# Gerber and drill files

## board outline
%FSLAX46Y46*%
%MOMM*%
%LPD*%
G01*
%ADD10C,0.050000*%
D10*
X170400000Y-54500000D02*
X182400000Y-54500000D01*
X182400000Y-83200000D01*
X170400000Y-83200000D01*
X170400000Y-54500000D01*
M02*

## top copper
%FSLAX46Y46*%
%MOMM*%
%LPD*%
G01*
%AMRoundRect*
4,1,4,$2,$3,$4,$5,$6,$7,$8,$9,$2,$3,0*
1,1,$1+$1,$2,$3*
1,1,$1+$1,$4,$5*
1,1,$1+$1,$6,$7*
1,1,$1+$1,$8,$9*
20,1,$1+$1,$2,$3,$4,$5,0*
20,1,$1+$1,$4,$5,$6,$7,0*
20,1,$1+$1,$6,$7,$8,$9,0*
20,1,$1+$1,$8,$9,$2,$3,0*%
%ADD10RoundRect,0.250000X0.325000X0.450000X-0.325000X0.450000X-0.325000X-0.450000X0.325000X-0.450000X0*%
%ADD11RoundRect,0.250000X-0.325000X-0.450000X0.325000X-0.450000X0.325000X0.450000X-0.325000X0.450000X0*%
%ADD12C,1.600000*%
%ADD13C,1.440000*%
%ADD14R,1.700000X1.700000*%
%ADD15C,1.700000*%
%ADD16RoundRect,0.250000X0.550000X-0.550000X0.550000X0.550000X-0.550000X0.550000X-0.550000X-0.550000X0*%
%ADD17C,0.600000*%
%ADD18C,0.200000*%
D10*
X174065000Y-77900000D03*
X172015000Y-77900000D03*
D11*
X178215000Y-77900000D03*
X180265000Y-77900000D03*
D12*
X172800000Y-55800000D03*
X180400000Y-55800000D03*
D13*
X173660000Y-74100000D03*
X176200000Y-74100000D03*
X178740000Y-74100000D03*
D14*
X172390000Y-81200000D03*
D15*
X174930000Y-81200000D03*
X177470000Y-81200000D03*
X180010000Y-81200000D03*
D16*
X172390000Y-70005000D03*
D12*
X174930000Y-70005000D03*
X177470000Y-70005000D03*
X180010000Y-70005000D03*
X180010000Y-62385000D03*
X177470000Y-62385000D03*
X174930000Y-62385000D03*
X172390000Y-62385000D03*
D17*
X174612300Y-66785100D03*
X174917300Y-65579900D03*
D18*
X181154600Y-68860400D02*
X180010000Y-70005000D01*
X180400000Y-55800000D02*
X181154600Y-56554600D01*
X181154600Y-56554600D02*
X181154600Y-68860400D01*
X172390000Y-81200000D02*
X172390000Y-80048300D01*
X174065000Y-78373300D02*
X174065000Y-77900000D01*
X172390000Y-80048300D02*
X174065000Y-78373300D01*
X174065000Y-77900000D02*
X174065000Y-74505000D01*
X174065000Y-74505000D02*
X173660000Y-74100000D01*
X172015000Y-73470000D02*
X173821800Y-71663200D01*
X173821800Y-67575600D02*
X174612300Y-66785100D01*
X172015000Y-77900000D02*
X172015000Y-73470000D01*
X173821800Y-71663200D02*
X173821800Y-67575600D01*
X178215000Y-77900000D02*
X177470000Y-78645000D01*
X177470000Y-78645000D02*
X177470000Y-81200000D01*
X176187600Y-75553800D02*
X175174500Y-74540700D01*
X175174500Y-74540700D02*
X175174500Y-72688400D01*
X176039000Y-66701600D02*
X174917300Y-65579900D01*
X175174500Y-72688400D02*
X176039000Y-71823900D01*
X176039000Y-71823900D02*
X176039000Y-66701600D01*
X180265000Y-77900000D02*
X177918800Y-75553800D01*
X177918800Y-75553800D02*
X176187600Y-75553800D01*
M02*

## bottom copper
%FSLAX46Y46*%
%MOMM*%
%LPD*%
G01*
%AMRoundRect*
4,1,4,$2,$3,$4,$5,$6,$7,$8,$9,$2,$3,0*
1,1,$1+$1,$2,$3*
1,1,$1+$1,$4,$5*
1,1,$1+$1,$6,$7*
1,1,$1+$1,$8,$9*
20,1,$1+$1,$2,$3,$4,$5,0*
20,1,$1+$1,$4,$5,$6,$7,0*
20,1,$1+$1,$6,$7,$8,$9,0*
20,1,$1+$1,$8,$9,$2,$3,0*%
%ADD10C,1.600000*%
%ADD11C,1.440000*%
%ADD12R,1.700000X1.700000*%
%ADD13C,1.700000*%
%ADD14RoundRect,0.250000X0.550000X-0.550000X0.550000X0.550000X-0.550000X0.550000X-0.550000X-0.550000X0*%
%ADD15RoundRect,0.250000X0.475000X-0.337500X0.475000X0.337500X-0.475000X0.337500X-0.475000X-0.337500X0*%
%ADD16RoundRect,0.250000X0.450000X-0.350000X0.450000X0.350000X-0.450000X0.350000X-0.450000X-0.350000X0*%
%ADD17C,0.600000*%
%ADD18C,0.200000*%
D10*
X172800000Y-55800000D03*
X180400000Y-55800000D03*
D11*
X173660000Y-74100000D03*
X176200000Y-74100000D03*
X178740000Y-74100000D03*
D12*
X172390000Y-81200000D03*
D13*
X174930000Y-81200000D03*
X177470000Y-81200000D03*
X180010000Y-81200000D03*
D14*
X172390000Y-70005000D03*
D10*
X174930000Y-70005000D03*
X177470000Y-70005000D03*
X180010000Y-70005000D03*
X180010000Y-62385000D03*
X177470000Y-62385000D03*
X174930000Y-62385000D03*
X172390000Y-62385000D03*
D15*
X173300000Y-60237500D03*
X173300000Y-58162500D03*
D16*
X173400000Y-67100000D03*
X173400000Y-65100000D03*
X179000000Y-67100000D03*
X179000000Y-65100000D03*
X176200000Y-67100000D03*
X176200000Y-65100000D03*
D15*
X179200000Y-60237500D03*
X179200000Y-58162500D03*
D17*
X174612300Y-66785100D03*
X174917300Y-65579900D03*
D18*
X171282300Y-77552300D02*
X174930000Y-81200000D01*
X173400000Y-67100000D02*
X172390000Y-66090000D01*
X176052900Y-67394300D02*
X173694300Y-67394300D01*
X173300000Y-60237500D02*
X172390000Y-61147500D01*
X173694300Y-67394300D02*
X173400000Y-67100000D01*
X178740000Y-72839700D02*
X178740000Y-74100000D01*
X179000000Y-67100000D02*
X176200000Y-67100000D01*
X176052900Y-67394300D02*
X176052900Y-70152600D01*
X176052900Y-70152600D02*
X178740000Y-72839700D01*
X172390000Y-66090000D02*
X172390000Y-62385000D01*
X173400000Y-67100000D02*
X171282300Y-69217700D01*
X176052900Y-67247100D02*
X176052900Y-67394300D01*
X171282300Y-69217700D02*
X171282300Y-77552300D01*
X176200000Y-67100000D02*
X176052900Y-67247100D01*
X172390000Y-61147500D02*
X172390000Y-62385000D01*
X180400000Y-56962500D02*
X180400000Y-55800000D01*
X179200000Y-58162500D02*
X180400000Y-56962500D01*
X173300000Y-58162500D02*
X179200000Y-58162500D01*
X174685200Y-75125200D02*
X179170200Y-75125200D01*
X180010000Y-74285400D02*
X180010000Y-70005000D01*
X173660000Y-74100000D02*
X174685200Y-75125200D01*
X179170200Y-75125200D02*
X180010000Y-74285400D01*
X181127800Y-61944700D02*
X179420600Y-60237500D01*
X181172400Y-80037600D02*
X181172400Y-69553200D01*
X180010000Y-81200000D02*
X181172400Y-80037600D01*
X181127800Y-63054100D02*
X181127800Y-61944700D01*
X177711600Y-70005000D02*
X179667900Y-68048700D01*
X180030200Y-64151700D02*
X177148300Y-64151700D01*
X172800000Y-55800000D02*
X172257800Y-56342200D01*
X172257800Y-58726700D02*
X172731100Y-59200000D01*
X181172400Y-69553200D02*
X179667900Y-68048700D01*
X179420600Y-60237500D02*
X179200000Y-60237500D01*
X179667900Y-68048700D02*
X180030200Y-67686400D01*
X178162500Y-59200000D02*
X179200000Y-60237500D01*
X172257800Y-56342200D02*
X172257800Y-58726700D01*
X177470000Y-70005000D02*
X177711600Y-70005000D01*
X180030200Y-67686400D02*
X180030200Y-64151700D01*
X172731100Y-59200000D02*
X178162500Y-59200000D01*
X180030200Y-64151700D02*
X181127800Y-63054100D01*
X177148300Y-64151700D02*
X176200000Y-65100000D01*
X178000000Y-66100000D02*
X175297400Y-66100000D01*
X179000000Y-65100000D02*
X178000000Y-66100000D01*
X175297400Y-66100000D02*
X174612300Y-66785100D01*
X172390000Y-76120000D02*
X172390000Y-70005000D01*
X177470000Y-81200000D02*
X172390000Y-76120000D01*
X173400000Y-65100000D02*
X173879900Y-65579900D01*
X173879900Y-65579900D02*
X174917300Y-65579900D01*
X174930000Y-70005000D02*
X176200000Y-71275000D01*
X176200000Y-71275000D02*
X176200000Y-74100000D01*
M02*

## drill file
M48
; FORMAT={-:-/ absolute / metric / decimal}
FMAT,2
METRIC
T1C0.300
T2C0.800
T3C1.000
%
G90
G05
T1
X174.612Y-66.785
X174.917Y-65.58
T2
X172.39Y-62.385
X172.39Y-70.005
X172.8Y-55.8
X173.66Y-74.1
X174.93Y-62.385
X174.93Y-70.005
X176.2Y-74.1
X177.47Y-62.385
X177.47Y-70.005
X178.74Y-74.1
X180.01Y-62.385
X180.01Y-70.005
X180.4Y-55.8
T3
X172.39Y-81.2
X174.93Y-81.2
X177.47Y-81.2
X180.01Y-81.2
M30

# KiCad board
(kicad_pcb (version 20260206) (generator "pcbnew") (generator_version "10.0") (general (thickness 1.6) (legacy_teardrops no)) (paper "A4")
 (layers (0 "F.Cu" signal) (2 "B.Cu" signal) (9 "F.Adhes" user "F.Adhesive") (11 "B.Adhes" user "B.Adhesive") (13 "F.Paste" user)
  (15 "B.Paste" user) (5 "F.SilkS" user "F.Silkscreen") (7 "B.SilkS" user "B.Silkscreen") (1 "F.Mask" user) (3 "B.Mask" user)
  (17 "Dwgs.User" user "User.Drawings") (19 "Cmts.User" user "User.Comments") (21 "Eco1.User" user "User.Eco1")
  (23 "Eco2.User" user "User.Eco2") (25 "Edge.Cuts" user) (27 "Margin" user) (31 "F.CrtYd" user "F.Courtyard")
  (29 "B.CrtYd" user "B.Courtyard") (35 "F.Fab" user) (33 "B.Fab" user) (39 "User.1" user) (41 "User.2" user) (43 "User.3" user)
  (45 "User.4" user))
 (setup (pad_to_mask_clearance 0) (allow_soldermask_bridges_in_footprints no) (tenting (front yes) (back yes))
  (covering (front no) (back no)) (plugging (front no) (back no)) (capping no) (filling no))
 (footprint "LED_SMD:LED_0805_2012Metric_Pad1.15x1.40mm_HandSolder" (layer "F.Cu") (at 173.04 77.9 180)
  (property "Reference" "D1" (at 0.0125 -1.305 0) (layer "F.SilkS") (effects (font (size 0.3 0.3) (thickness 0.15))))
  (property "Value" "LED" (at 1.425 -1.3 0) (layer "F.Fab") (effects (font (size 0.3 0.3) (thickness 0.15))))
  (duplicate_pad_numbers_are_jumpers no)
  (pad "1" smd roundrect (at -1.025 0 180) (size 1.15 1.4) (layers "F.Cu" "F.Mask" "F.Paste") (roundrect_rratio 0.217391) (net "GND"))
  (pad "2" smd roundrect (at 1.025 0 180) (size 1.15 1.4) (layers "F.Cu" "F.Mask" "F.Paste") (roundrect_rratio 0.217391) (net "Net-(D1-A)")))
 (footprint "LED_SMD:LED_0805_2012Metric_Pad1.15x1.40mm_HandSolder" (layer "F.Cu") (at 179.24 77.9)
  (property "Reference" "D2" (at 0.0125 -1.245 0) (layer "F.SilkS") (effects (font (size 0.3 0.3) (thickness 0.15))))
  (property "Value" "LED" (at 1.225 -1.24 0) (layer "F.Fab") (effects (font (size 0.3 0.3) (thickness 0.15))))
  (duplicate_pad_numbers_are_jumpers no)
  (pad "1" smd roundrect (at -1.025 0) (size 1.15 1.4) (layers "F.Cu" "F.Mask" "F.Paste") (roundrect_rratio 0.217391) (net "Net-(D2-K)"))
  (pad "2" smd roundrect (at 1.025 0) (size 1.15 1.4) (layers "F.Cu" "F.Mask" "F.Paste") (roundrect_rratio 0.217391) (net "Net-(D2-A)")))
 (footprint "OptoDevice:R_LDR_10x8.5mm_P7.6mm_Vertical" (layer "F.Cu") (at 172.8 55.8)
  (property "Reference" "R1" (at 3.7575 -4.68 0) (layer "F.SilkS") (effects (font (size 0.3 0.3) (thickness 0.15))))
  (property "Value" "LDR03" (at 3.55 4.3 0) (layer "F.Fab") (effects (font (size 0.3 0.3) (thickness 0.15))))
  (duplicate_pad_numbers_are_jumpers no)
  (pad "1" thru_hole circle (at 0 0) (size 1.6 1.6) (drill 0.8) (layers "*.Cu" "*.Mask") (remove_unused_layers no) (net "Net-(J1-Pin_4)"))
  (pad "2" thru_hole circle (at 7.6 0) (size 1.6 1.6) (drill 0.8) (layers "*.Cu" "*.Mask") (remove_unused_layers no) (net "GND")))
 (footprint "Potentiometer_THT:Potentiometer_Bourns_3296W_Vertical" (layer "F.Cu") (at 173.66 74.1 180)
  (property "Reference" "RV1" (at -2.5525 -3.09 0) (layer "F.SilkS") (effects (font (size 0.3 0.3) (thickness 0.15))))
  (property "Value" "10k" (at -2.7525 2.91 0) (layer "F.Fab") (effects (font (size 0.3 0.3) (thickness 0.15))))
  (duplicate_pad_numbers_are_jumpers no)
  (pad "1" thru_hole circle (at 0 0 180) (size 1.44 1.44) (drill 0.8) (layers "*.Cu" "*.Mask") (remove_unused_layers no) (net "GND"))
  (pad "2" thru_hole circle (at -2.54 0 180) (size 1.44 1.44) (drill 0.8) (layers "*.Cu" "*.Mask") (remove_unused_layers no)
   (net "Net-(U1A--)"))
  (pad "3" thru_hole circle (at -5.08 0 180) (size 1.44 1.44) (drill 0.8) (layers "*.Cu" "*.Mask") (remove_unused_layers no) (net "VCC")))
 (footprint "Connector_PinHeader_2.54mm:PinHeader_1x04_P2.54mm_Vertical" (layer "F.Cu") (at 172.39 81.2 90)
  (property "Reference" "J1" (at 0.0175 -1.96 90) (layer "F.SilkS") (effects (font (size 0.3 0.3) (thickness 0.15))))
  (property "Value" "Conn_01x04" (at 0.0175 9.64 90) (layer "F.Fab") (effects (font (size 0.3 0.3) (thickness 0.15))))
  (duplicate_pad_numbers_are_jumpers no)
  (pad "1" thru_hole rect (at 0 0 90) (size 1.7 1.7) (drill 1) (layers "*.Cu" "*.Mask") (remove_unused_layers no) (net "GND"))
  (pad "2" thru_hole circle (at 0 2.54 90) (size 1.7 1.7) (drill 1) (layers "*.Cu" "*.Mask") (remove_unused_layers no) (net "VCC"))
  (pad "3" thru_hole circle (at 0 5.08 90) (size 1.7 1.7) (drill 1) (layers "*.Cu" "*.Mask") (remove_unused_layers no) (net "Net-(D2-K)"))
  (pad "4" thru_hole circle (at 0 7.62 90) (size 1.7 1.7) (drill 1) (layers "*.Cu" "*.Mask") (remove_unused_layers no)
   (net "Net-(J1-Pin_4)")))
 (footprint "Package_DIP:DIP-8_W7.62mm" (layer "F.Cu") (at 172.39 70.005 90)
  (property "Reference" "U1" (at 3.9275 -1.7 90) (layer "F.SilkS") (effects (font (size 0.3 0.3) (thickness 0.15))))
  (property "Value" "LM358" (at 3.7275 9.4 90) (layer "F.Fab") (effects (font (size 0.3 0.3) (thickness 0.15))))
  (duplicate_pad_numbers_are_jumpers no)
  (pad "1" thru_hole roundrect (at 0 0 90) (size 1.6 1.6) (drill 0.8) (layers "*.Cu" "*.Mask") (remove_unused_layers no)
   (roundrect_rratio 0.15625) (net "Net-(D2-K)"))
  (pad "2" thru_hole circle (at 0 2.54 90) (size 1.6 1.6) (drill 0.8) (layers "*.Cu" "*.Mask") (remove_unused_layers no) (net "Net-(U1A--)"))
  (pad "3" thru_hole circle (at 0 5.08 90) (size 1.6 1.6) (drill 0.8) (layers "*.Cu" "*.Mask") (remove_unused_layers no)
   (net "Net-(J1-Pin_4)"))
  (pad "4" thru_hole circle (at 0 7.62 90) (size 1.6 1.6) (drill 0.8) (layers "*.Cu" "*.Mask") (remove_unused_layers no) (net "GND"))
  (pad "5" thru_hole circle (at 7.62 7.62 90) (size 1.6 1.6) (drill 0.8) (layers "*.Cu" "*.Mask") (remove_unused_layers no))
  (pad "6" thru_hole circle (at 7.62 5.08 90) (size 1.6 1.6) (drill 0.8) (layers "*.Cu" "*.Mask") (remove_unused_layers no))
  (pad "7" thru_hole circle (at 7.62 2.54 90) (size 1.6 1.6) (drill 0.8) (layers "*.Cu" "*.Mask") (remove_unused_layers no))
  (pad "8" thru_hole circle (at 7.62 0 90) (size 1.6 1.6) (drill 0.8) (layers "*.Cu" "*.Mask") (remove_unused_layers no) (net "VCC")))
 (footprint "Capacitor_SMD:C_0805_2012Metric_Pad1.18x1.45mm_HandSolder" (layer "B.Cu") (at 173.3 59.2 90)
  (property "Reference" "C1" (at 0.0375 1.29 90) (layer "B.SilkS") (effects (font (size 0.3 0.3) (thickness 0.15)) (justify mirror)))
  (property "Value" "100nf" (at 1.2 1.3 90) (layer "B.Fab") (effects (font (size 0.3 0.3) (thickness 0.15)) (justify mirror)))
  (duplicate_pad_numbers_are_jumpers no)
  (pad "1" smd roundrect (at -1.0375 0 90) (size 1.175 1.45) (layers "B.Cu" "B.Mask" "B.Paste") (roundrect_rratio 0.212766) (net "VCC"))
  (pad "2" smd roundrect (at 1.0375 0 90) (size 1.175 1.45) (layers "B.Cu" "B.Mask" "B.Paste") (roundrect_rratio 0.212766) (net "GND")))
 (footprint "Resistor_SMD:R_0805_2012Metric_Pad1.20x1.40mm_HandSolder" (layer "B.Cu") (at 173.4 66.1 90)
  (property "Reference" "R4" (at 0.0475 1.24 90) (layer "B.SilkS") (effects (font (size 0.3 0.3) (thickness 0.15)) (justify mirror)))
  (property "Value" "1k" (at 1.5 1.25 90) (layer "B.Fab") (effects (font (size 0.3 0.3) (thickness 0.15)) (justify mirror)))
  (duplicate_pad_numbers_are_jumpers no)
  (pad "1" smd roundrect (at -1 0 90) (size 1.2 1.4) (layers "B.Cu" "B.Mask" "B.Paste") (roundrect_rratio 0.208333) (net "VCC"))
  (pad "2" smd roundrect (at 1 0 90) (size 1.2 1.4) (layers "B.Cu" "B.Mask" "B.Paste") (roundrect_rratio 0.208333) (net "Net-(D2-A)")))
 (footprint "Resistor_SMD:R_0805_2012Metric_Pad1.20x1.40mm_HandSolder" (layer "B.Cu") (at 179 66.1 90)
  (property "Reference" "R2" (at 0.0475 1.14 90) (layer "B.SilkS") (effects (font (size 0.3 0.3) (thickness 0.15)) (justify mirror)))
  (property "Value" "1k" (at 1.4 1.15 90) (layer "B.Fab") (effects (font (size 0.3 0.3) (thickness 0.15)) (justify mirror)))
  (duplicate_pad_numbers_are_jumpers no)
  (pad "1" smd roundrect (at -1 0 90) (size 1.2 1.4) (layers "B.Cu" "B.Mask" "B.Paste") (roundrect_rratio 0.208333) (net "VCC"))
  (pad "2" smd roundrect (at 1 0 90) (size 1.2 1.4) (layers "B.Cu" "B.Mask" "B.Paste") (roundrect_rratio 0.208333) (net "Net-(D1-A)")))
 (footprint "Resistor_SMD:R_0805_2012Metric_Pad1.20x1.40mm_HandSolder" (layer "B.Cu") (at 176.2 66.1 90)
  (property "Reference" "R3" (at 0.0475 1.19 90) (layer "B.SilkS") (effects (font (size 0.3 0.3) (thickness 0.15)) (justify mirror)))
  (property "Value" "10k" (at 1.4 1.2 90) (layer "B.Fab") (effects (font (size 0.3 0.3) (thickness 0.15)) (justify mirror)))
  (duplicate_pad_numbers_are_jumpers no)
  (pad "1" smd roundrect (at -1 0 90) (size 1.2 1.4) (layers "B.Cu" "B.Mask" "B.Paste") (roundrect_rratio 0.208333) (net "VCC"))
  (pad "2" smd roundrect (at 1 0 90) (size 1.2 1.4) (layers "B.Cu" "B.Mask" "B.Paste") (roundrect_rratio 0.208333) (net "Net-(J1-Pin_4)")))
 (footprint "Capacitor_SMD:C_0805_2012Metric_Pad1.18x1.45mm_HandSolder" (layer "B.Cu") (at 179.2 59.2 90)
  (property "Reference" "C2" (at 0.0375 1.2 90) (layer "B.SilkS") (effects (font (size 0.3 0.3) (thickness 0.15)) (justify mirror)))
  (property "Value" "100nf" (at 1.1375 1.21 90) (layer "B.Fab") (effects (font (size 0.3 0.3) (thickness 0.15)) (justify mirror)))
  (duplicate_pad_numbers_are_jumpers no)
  (pad "1" smd roundrect (at -1.0375 0 90) (size 1.175 1.45) (layers "B.Cu" "B.Mask" "B.Paste") (roundrect_rratio 0.212766)
   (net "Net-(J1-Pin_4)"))
  (pad "2" smd roundrect (at 1.0375 0 90) (size 1.175 1.45) (layers "B.Cu" "B.Mask" "B.Paste") (roundrect_rratio 0.212766) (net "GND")))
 (gr_rect (start 170.4 54.5) (end 182.4 83.2) (stroke (width 0.05) (type default)) (fill no) (layer "Edge.Cuts"))
 (segment (start 171.2823 77.5523) (end 174.93 81.2) (width 0.2) (layer "B.Cu") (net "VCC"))
 (segment (start 173.4 67.1) (end 172.39 66.09) (width 0.2) (layer "B.Cu") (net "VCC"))
 (segment (start 176.0529 67.3943) (end 173.6943 67.3943) (width 0.2) (layer "B.Cu") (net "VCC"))
 (segment (start 173.3 60.2375) (end 172.39 61.1475) (width 0.2) (layer "B.Cu") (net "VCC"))
 (segment (start 173.6943 67.3943) (end 173.4 67.1) (width 0.2) (layer "B.Cu") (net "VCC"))
 (segment (start 178.74 72.8397) (end 178.74 74.1) (width 0.2) (layer "B.Cu") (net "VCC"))
 (segment (start 179 67.1) (end 176.2 67.1) (width 0.2) (layer "B.Cu") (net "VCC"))
 (segment (start 176.0529 67.3943) (end 176.0529 70.1526) (width 0.2) (layer "B.Cu") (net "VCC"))
 (segment (start 176.0529 70.1526) (end 178.74 72.8397) (width 0.2) (layer "B.Cu") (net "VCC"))
 (segment (start 172.39 66.09) (end 172.39 62.385) (width 0.2) (layer "B.Cu") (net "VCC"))
 (segment (start 173.4 67.1) (end 171.2823 69.2177) (width 0.2) (layer "B.Cu") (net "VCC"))
 (segment (start 176.0529 67.2471) (end 176.0529 67.3943) (width 0.2) (layer "B.Cu") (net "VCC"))
 (segment (start 171.2823 69.2177) (end 171.2823 77.5523) (width 0.2) (layer "B.Cu") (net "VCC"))
 (segment (start 176.2 67.1) (end 176.0529 67.2471) (width 0.2) (layer "B.Cu") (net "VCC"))
 (segment (start 172.39 61.1475) (end 172.39 62.385) (width 0.2) (layer "B.Cu") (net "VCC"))
 (segment (start 181.1546 68.8604) (end 180.01 70.005) (width 0.2) (layer "F.Cu") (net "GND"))
 (segment (start 180.4 55.8) (end 181.1546 56.5546) (width 0.2) (layer "F.Cu") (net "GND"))
 (segment (start 181.1546 56.5546) (end 181.1546 68.8604) (width 0.2) (layer "F.Cu") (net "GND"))
 (segment (start 172.39 81.2) (end 172.39 80.0483) (width 0.2) (layer "F.Cu") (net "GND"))
 (segment (start 174.065 78.3733) (end 174.065 77.9) (width 0.2) (layer "F.Cu") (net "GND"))
 (segment (start 172.39 80.0483) (end 174.065 78.3733) (width 0.2) (layer "F.Cu") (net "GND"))
 (segment (start 174.065 77.9) (end 174.065 74.505) (width 0.2) (layer "F.Cu") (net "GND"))
 (segment (start 174.065 74.505) (end 173.66 74.1) (width 0.2) (layer "F.Cu") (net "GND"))
 (segment (start 180.4 56.9625) (end 180.4 55.8) (width 0.2) (layer "B.Cu") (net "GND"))
 (segment (start 179.2 58.1625) (end 180.4 56.9625) (width 0.2) (layer "B.Cu") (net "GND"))
 (segment (start 173.3 58.1625) (end 179.2 58.1625) (width 0.2) (layer "B.Cu") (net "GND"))
 (segment (start 174.6852 75.1252) (end 179.1702 75.1252) (width 0.2) (layer "B.Cu") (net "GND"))
 (segment (start 180.01 74.2854) (end 180.01 70.005) (width 0.2) (layer "B.Cu") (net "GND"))
 (segment (start 173.66 74.1) (end 174.6852 75.1252) (width 0.2) (layer "B.Cu") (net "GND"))
 (segment (start 179.1702 75.1252) (end 180.01 74.2854) (width 0.2) (layer "B.Cu") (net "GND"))
 (segment (start 181.1278 61.9447) (end 179.4206 60.2375) (width 0.2) (layer "B.Cu") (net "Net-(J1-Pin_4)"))
 (segment (start 181.1724 80.0376) (end 181.1724 69.5532) (width 0.2) (layer "B.Cu") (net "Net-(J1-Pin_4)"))
 (segment (start 180.01 81.2) (end 181.1724 80.0376) (width 0.2) (layer "B.Cu") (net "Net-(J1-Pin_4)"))
 (segment (start 181.1278 63.0541) (end 181.1278 61.9447) (width 0.2) (layer "B.Cu") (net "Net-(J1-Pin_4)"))
 (segment (start 177.7116 70.005) (end 179.6679 68.0487) (width 0.2) (layer "B.Cu") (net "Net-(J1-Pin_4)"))
 (segment (start 180.0302 64.1517) (end 177.1483 64.1517) (width 0.2) (layer "B.Cu") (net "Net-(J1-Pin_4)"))
 (segment (start 172.8 55.8) (end 172.2578 56.3422) (width 0.2) (layer "B.Cu") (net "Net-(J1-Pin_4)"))
 (segment (start 172.2578 58.7267) (end 172.7311 59.2) (width 0.2) (layer "B.Cu") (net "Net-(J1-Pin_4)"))
 (segment (start 181.1724 69.5532) (end 179.6679 68.0487) (width 0.2) (layer "B.Cu") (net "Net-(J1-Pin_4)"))
 (segment (start 179.4206 60.2375) (end 179.2 60.2375) (width 0.2) (layer "B.Cu") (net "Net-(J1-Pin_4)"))
 (segment (start 179.6679 68.0487) (end 180.0302 67.6864) (width 0.2) (layer "B.Cu") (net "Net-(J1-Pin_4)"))
 (segment (start 178.1625 59.2) (end 179.2 60.2375) (width 0.2) (layer "B.Cu") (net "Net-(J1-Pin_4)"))
 (segment (start 172.2578 56.3422) (end 172.2578 58.7267) (width 0.2) (layer "B.Cu") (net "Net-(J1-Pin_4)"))
 (segment (start 177.47 70.005) (end 177.7116 70.005) (width 0.2) (layer "B.Cu") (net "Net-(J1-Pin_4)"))
 (segment (start 180.0302 67.6864) (end 180.0302 64.1517) (width 0.2) (layer "B.Cu") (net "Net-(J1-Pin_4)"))
 (segment (start 172.7311 59.2) (end 178.1625 59.2) (width 0.2) (layer "B.Cu") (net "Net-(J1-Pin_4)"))
 (segment (start 180.0302 64.1517) (end 181.1278 63.0541) (width 0.2) (layer "B.Cu") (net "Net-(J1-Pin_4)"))
 (segment (start 177.1483 64.1517) (end 176.2 65.1) (width 0.2) (layer "B.Cu") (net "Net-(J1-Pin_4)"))
 (segment (start 172.015 73.47) (end 173.8218 71.6632) (width 0.2) (layer "F.Cu") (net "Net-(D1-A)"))
 (segment (start 173.8218 67.5756) (end 174.6123 66.7851) (width 0.2) (layer "F.Cu") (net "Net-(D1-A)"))
 (segment (start 172.015 77.9) (end 172.015 73.47) (width 0.2) (layer "F.Cu") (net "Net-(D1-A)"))
 (segment (start 173.8218 71.6632) (end 173.8218 67.5756) (width 0.2) (layer "F.Cu") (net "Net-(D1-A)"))
 (via (at 174.6123 66.7851) (size 0.6) (drill 0.3) (layers "F.Cu" "B.Cu") (capping no) (covering (front no) (back no))
  (plugging (front no) (back no)) (filling no) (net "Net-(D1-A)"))
 (segment (start 178 66.1) (end 175.2974 66.1) (width 0.2) (layer "B.Cu") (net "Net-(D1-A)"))
 (segment (start 179 65.1) (end 178 66.1) (width 0.2) (layer "B.Cu") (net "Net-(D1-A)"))
 (segment (start 175.2974 66.1) (end 174.6123 66.7851) (width 0.2) (layer "B.Cu") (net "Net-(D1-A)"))
 (segment (start 178.215 77.9) (end 177.47 78.645) (width 0.2) (layer "F.Cu") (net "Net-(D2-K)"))
 (segment (start 177.47 78.645) (end 177.47 81.2) (width 0.2) (layer "F.Cu") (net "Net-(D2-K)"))
 (segment (start 172.39 76.12) (end 172.39 70.005) (width 0.2) (layer "B.Cu") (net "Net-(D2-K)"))
 (segment (start 177.47 81.2) (end 172.39 76.12) (width 0.2) (layer "B.Cu") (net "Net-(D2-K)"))
 (segment (start 176.1876 75.5538) (end 175.1745 74.5407) (width 0.2) (layer "F.Cu") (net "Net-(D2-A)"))
 (segment (start 175.1745 74.5407) (end 175.1745 72.6884) (width 0.2) (layer "F.Cu") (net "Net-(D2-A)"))
 (segment (start 176.039 66.7016) (end 174.9173 65.5799) (width 0.2) (layer "F.Cu") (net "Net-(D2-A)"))
 (segment (start 175.1745 72.6884) (end 176.039 71.8239) (width 0.2) (layer "F.Cu") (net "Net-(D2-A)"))
 (segment (start 176.039 71.8239) (end 176.039 66.7016) (width 0.2) (layer "F.Cu") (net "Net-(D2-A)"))
 (segment (start 180.265 77.9) (end 177.9188 75.5538) (width 0.2) (layer "F.Cu") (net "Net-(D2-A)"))
 (segment (start 177.9188 75.5538) (end 176.1876 75.5538) (width 0.2) (layer "F.Cu") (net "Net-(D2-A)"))
 (via (at 174.9173 65.5799) (size 0.6) (drill 0.3) (layers "F.Cu" "B.Cu") (capping no) (covering (front no) (back no))
  (plugging (front no) (back no)) (filling no) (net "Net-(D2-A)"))
 (segment (start 173.4 65.1) (end 173.8799 65.5799) (width 0.2) (layer "B.Cu") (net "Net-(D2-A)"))
 (segment (start 173.8799 65.5799) (end 174.9173 65.5799) (width 0.2) (layer "B.Cu") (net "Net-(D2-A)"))
 (segment (start 174.93 70.005) (end 176.2 71.275) (width 0.2) (layer "B.Cu") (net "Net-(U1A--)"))
 (segment (start 176.2 71.275) (end 176.2 74.1) (width 0.2) (layer "B.Cu") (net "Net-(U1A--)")))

